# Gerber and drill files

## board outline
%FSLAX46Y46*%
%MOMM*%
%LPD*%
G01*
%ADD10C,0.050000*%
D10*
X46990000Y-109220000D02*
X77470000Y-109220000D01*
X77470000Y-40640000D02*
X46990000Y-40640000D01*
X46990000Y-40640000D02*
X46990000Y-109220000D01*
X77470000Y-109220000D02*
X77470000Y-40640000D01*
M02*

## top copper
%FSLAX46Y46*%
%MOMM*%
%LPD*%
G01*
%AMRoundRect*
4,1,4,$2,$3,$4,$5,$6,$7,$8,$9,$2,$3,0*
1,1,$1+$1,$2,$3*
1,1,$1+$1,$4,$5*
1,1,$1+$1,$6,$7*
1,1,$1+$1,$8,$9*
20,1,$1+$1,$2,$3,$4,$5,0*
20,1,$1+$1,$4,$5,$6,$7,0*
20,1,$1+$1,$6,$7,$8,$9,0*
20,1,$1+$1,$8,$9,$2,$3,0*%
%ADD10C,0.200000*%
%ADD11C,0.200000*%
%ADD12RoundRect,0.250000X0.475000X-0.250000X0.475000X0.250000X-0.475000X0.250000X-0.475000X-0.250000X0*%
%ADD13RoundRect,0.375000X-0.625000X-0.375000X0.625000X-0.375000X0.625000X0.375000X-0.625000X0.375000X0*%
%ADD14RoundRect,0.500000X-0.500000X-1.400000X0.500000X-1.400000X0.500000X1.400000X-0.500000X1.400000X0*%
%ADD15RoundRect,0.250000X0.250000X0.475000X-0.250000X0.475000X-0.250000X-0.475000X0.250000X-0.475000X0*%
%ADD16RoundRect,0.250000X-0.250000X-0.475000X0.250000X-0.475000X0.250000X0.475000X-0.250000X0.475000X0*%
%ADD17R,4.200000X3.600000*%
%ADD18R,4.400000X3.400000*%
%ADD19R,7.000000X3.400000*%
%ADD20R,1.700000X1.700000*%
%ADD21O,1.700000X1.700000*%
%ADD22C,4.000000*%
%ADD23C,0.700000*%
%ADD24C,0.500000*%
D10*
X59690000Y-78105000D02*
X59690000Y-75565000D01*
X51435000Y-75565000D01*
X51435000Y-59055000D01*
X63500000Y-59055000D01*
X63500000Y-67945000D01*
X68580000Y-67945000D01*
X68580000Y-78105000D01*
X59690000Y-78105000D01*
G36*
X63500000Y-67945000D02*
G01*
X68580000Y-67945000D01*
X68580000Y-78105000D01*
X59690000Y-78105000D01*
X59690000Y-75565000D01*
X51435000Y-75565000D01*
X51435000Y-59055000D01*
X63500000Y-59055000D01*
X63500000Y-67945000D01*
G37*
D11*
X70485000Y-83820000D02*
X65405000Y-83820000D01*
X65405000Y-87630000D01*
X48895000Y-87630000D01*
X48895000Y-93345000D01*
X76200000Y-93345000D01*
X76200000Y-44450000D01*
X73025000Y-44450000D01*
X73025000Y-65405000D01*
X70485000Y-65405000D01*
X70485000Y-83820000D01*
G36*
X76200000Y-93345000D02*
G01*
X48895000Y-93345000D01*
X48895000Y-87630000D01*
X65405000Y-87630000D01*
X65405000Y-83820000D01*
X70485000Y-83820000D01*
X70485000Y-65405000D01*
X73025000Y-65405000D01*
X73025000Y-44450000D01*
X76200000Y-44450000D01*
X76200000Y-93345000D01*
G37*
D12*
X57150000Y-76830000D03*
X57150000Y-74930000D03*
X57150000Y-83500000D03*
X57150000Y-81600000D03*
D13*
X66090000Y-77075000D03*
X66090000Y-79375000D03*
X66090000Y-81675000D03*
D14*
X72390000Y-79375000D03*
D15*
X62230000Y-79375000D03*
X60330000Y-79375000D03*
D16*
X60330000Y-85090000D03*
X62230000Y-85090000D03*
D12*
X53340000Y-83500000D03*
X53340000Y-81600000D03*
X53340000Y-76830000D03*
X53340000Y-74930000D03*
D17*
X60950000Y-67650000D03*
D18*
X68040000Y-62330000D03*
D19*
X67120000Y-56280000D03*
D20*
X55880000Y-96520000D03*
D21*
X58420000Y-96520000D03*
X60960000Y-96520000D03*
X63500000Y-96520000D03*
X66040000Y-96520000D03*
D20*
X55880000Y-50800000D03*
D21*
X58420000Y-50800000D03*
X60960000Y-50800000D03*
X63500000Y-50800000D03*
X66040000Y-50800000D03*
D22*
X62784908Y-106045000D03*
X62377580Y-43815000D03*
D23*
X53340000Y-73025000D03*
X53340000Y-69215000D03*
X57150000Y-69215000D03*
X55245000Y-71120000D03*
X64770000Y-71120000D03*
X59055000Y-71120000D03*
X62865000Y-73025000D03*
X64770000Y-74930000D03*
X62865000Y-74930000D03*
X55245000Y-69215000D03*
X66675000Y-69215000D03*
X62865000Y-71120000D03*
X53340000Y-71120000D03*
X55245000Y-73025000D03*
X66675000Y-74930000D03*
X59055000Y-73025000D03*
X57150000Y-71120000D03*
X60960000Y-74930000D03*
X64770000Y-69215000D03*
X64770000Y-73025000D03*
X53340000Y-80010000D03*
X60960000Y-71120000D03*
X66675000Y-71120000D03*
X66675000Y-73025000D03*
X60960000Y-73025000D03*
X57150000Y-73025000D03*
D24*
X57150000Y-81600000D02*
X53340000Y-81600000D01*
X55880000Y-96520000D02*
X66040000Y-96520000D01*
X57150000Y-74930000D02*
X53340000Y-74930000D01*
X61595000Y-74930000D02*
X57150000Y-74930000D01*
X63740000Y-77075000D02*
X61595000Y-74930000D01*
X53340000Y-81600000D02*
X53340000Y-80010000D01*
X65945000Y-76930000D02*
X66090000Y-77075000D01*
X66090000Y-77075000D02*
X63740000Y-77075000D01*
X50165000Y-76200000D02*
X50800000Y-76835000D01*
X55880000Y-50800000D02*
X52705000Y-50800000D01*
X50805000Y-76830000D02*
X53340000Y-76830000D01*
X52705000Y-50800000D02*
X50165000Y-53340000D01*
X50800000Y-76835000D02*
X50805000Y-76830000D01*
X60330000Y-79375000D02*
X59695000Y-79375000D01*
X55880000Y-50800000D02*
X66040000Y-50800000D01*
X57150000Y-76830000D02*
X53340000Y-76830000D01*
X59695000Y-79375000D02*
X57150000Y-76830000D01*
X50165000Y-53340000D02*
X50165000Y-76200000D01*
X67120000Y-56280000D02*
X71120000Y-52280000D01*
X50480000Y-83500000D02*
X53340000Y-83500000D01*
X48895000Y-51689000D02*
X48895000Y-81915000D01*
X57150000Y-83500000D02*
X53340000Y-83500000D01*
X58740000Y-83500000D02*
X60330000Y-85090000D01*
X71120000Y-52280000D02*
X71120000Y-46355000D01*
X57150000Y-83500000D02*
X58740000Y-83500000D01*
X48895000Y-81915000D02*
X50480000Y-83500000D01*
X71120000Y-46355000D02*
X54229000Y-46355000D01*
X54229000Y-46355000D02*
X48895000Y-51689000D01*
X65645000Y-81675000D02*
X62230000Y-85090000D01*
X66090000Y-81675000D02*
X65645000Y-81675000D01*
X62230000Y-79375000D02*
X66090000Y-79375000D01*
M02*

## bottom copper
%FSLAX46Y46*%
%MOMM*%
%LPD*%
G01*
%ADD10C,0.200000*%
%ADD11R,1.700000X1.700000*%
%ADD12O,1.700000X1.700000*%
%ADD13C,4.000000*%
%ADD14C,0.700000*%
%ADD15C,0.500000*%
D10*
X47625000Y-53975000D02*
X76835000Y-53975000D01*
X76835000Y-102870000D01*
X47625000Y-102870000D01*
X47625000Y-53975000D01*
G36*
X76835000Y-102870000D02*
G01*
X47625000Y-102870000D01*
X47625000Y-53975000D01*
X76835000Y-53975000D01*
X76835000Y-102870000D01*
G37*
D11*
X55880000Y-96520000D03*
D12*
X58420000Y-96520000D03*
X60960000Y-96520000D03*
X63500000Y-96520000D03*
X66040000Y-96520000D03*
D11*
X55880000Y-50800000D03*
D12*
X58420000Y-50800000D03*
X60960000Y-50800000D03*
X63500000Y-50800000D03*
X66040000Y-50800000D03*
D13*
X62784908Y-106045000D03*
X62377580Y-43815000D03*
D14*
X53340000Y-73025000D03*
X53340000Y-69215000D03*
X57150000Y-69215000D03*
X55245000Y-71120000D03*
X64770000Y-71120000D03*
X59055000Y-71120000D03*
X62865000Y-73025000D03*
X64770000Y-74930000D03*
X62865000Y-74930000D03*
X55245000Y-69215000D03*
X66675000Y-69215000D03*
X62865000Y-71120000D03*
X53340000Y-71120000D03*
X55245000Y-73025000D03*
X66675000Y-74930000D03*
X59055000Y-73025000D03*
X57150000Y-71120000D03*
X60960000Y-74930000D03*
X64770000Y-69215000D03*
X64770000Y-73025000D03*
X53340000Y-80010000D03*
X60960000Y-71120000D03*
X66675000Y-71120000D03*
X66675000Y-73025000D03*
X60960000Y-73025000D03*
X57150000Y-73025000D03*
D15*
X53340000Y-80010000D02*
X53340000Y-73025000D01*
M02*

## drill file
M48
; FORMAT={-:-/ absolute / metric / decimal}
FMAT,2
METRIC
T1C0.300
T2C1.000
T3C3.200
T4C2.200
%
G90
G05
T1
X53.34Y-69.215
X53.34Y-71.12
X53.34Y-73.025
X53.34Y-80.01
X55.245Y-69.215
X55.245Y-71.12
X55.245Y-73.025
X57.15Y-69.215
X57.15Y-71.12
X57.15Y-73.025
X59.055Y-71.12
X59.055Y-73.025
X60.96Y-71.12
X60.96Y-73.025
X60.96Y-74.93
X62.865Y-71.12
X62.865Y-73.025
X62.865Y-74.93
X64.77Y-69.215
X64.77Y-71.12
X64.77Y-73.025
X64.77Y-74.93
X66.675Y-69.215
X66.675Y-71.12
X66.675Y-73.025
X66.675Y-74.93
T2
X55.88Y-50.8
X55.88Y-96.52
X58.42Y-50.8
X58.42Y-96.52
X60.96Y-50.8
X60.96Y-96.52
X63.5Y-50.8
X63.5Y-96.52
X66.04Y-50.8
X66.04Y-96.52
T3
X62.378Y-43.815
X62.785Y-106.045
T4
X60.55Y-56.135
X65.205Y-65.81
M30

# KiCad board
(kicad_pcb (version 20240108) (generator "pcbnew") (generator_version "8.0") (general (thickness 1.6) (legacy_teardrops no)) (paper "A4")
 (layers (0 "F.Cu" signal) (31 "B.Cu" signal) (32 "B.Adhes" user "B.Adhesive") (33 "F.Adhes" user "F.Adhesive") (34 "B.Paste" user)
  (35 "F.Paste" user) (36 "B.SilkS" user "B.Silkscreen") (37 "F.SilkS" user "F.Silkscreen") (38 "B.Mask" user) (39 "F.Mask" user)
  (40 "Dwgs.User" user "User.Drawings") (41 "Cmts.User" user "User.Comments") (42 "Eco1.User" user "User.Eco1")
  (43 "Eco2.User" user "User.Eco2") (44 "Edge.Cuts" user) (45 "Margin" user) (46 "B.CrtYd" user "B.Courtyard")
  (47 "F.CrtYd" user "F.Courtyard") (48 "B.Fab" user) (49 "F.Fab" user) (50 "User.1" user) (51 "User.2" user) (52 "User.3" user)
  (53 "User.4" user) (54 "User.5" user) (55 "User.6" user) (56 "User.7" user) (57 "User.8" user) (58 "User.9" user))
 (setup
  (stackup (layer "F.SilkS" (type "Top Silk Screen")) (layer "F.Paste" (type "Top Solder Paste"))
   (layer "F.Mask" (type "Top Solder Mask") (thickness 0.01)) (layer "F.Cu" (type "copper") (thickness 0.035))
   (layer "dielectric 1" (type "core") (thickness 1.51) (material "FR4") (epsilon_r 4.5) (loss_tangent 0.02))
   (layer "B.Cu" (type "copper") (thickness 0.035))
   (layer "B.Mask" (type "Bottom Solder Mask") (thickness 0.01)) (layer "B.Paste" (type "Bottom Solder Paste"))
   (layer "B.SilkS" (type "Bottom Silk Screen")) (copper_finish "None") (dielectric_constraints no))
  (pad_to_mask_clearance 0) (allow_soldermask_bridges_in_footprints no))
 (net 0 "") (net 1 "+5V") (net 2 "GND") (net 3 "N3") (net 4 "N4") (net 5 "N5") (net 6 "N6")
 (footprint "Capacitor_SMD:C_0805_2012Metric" (layer "F.Cu") (at 57.15 75.88 90)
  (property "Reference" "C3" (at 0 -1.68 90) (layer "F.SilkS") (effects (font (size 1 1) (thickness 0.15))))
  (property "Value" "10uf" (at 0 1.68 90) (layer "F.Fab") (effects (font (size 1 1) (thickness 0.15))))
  (pad "1" smd roundrect (at -0.95 0 90) (size 1 1.45) (layers "F.Cu" "F.Paste" "F.Mask") (roundrect_rratio 0.25) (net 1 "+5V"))
  (pad "2" smd roundrect (at 0.95 0 90) (size 1 1.45) (layers "F.Cu" "F.Paste" "F.Mask") (roundrect_rratio 0.25) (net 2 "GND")))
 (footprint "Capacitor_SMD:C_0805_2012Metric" (layer "F.Cu") (at 57.15 82.55 90)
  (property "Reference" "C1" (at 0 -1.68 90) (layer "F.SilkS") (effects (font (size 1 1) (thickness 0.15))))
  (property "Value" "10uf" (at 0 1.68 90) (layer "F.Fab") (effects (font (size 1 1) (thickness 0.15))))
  (pad "1" smd roundrect (at -0.95 0 90) (size 1 1.45) (layers "F.Cu" "F.Paste" "F.Mask") (roundrect_rratio 0.25) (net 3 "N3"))
  (pad "2" smd roundrect (at 0.95 0 90) (size 1 1.45) (layers "F.Cu" "F.Paste" "F.Mask") (roundrect_rratio 0.25) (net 2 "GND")))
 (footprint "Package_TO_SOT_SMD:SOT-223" (layer "F.Cu") (at 69.24 79.375)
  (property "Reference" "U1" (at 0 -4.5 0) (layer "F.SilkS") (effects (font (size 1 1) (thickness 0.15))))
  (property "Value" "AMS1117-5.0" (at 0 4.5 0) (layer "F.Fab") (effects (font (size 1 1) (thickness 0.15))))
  (pad "1" smd roundrect (at -3.15 -2.3) (size 2 1.5) (layers "F.Cu" "F.Paste" "F.Mask") (roundrect_rratio 0.25) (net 2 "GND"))
  (pad "2" smd roundrect (at -3.15 0) (size 2 1.5) (layers "F.Cu" "F.Paste" "F.Mask") (roundrect_rratio 0.25) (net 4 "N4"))
  (pad "3" smd roundrect (at -3.15 2.3) (size 2 1.5) (layers "F.Cu" "F.Paste" "F.Mask") (roundrect_rratio 0.25) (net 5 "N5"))
  (pad "4" smd roundrect (at 3.15 0) (size 2 3.8) (layers "F.Cu" "F.Paste" "F.Mask") (roundrect_rratio 0.25)))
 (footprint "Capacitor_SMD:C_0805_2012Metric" (layer "F.Cu") (at 61.28 79.375 180)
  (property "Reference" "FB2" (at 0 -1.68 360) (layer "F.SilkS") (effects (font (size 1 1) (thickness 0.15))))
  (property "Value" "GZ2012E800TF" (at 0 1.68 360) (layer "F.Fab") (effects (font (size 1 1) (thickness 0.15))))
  (pad "1" smd roundrect (at -0.95 0 180) (size 1 1.45) (layers "F.Cu" "F.Paste" "F.Mask") (roundrect_rratio 0.25) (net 4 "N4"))
  (pad "2" smd roundrect (at 0.95 0 180) (size 1 1.45) (layers "F.Cu" "F.Paste" "F.Mask") (roundrect_rratio 0.25) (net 1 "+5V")))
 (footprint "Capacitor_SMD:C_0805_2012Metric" (layer "F.Cu") (at 61.28 85.09)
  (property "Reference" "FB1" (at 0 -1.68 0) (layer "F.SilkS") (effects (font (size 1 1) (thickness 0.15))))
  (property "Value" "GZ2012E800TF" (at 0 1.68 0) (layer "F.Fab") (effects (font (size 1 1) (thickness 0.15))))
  (pad "1" smd roundrect (at -0.95 0) (size 1 1.45) (layers "F.Cu" "F.Paste" "F.Mask") (roundrect_rratio 0.25) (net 3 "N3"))
  (pad "2" smd roundrect (at 0.95 0) (size 1 1.45) (layers "F.Cu" "F.Paste" "F.Mask") (roundrect_rratio 0.25) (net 5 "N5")))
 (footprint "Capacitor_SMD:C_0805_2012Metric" (layer "F.Cu") (at 53.34 82.55 90)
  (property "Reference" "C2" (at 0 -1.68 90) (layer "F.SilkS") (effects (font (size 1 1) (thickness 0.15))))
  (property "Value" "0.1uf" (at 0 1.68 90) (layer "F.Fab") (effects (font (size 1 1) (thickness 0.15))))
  (pad "1" smd roundrect (at -0.95 0 90) (size 1 1.45) (layers "F.Cu" "F.Paste" "F.Mask") (roundrect_rratio 0.25) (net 3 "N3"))
  (pad "2" smd roundrect (at 0.95 0 90) (size 1 1.45) (layers "F.Cu" "F.Paste" "F.Mask") (roundrect_rratio 0.25) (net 2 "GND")))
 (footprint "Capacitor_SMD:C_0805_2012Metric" (layer "F.Cu") (at 53.34 75.88 90)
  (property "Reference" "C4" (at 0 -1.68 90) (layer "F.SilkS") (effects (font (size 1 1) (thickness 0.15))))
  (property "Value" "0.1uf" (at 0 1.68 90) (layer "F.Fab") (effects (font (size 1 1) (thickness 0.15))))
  (pad "1" smd roundrect (at -0.95 0 90) (size 1 1.45) (layers "F.Cu" "F.Paste" "F.Mask") (roundrect_rratio 0.25) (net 1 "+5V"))
  (pad "2" smd roundrect (at 0.95 0 90) (size 1 1.45) (layers "F.Cu" "F.Paste" "F.Mask") (roundrect_rratio 0.25) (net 2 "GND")))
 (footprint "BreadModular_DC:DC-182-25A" (layer "F.Cu") (at 68.37 57.67 180)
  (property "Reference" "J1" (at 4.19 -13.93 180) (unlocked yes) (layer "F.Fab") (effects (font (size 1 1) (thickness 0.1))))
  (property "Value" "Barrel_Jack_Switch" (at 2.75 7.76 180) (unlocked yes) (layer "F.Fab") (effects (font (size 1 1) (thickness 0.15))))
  (pad "" np_thru_hole circle (at 3.165 -8.14 90) (size 2.2 2.2) (drill 2.2) (layers "F&B.Cu" "*.Mask"))
  (pad "" np_thru_hole circle (at 7.82 1.535 90) (size 2.2 2.2) (drill 2.2) (layers "F&B.Cu" "*.Mask"))
  (pad "1" smd rect (at 7.42 -9.98 90) (size 3.6 4.2) (layers "F.Cu" "F.Paste" "F.Mask") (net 2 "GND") (thermal_bridge_angle 45))
  (pad "2" smd rect (at 0.33 -4.66 90) (size 3.4 4.4) (layers "F.Cu" "F.Paste" "F.Mask") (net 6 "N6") (thermal_bridge_angle 45))
  (pad "3" smd rect (at 1.25 1.39 90) (size 3.4 7) (layers "F.Cu" "F.Paste" "F.Mask") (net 3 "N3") (thermal_bridge_angle 45)))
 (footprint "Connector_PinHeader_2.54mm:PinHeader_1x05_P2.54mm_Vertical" (layer "B.Cu") (at 55.88 96.52 -90)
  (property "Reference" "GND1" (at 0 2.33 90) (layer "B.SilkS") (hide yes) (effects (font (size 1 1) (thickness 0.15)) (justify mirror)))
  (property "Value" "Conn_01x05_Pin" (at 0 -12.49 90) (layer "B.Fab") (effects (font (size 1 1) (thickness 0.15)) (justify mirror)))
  (pad "1" thru_hole rect (at 0 0 270) (size 1.7 1.7) (drill 1) (layers "*.Cu" "*.Mask") (remove_unused_layers no) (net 2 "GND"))
  (pad "2" thru_hole oval (at 0 -2.54 270) (size 1.7 1.7) (drill 1) (layers "*.Cu" "*.Mask") (remove_unused_layers no) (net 2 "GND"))
  (pad "3" thru_hole oval (at 0 -5.08 270) (size 1.7 1.7) (drill 1) (layers "*.Cu" "*.Mask") (remove_unused_layers no) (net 2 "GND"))
  (pad "4" thru_hole oval (at 0 -7.62 270) (size 1.7 1.7) (drill 1) (layers "*.Cu" "*.Mask") (remove_unused_layers no) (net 2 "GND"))
  (pad "5" thru_hole oval (at 0 -10.16 270) (size 1.7 1.7) (drill 1) (layers "*.Cu" "*.Mask") (remove_unused_layers no) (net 2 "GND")))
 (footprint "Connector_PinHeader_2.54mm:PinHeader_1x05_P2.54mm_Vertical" (layer "B.Cu") (at 55.88 50.8 -90)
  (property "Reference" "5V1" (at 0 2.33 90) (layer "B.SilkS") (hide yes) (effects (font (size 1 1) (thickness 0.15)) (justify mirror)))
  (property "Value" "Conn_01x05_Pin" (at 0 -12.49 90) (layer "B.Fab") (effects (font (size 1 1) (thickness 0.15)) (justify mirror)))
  (pad "1" thru_hole rect (at 0 0 270) (size 1.7 1.7) (drill 1) (layers "*.Cu" "*.Mask") (remove_unused_layers no) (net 1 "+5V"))
  (pad "2" thru_hole oval (at 0 -2.54 270) (size 1.7 1.7) (drill 1) (layers "*.Cu" "*.Mask") (remove_unused_layers no) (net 1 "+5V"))
  (pad "3" thru_hole oval (at 0 -5.08 270) (size 1.7 1.7) (drill 1) (layers "*.Cu" "*.Mask") (remove_unused_layers no) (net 1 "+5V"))
  (pad "4" thru_hole oval (at 0 -7.62 270) (size 1.7 1.7) (drill 1) (layers "*.Cu" "*.Mask") (remove_unused_layers no) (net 1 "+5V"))
  (pad "5" thru_hole oval (at 0 -10.16 270) (size 1.7 1.7) (drill 1) (layers "*.Cu" "*.Mask") (remove_unused_layers no) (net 1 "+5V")))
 (gr_poly
  (pts (xy 59.69 78.105) (xy 59.69 75.565) (xy 51.435 75.565) (xy 51.435 59.055) (xy 63.5 59.055) (xy 63.5 67.945) (xy 68.58 67.945)
   (xy 68.58 78.105))
  (stroke (width 0.2) (type solid)) (fill solid) (layer "F.Cu") (net 2))
 (gr_poly
  (pts (xy 70.485 83.82) (xy 65.405 83.82) (xy 65.405 87.63) (xy 48.895 87.63) (xy 48.895 93.345) (xy 76.2 93.345) (xy 76.2 44.45)
   (xy 73.025 44.45) (xy 73.025 65.405) (xy 70.485 65.405))
  (stroke (width 0.2) (type solid)) (fill solid) (layer "F.Cu"))
 (gr_poly
  (pts (xy 47.625 53.975) (xy 76.835 53.975) (xy 76.835 102.87) (xy 47.625 102.87)) (stroke (width 0.2) (type solid)) (fill solid)
  (layer "B.Cu") (net 2))
 (gr_line (start 46.99 109.22) (end 77.47 109.22) (stroke (width 0.05) (type default)) (layer "Edge.Cuts"))
 (gr_line (start 77.47 40.64) (end 46.99 40.64) (stroke (width 0.05) (type default)) (layer "Edge.Cuts"))
 (gr_line (start 46.99 40.64) (end 46.99 109.22) (stroke (width 0.05) (type default)) (layer "Edge.Cuts"))
 (gr_line (start 77.47 109.22) (end 77.47 40.64) (stroke (width 0.05) (type default)) (layer "Edge.Cuts"))
 (via (at 62.784908 106.045) (size 4) (drill 3.2) (layers "F.Cu" "B.Cu") (free yes) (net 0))
 (via (at 62.37758 43.815) (size 4) (drill 3.2) (layers "F.Cu" "B.Cu") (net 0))
 (segment (start 57.15 81.6) (end 53.34 81.6) (width 0.5) (layer "F.Cu") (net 2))
 (segment (start 55.88 96.52) (end 66.04 96.52) (width 0.5) (layer "F.Cu") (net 2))
 (segment (start 57.15 74.93) (end 53.34 74.93) (width 0.5) (layer "F.Cu") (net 2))
 (segment (start 61.595 74.93) (end 57.15 74.93) (width 0.5) (layer "F.Cu") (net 2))
 (segment (start 63.74 77.075) (end 61.595 74.93) (width 0.5) (layer "F.Cu") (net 2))
 (segment (start 53.34 81.6) (end 53.34 80.01) (width 0.5) (layer "F.Cu") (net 2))
 (segment (start 65.945 76.93) (end 66.09 77.075) (width 0.5) (layer "F.Cu") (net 2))
 (segment (start 66.09 77.075) (end 63.74 77.075) (width 0.5) (layer "F.Cu") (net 2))
 (via (at 53.34 73.025) (size 0.7) (drill 0.3) (layers "F.Cu" "B.Cu") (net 2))
 (via (at 53.34 69.215) (size 0.7) (drill 0.3) (layers "F.Cu" "B.Cu") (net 2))
 (via (at 57.15 69.215) (size 0.7) (drill 0.3) (layers "F.Cu" "B.Cu") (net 2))
 (via (at 55.245 71.12) (size 0.7) (drill 0.3) (layers "F.Cu" "B.Cu") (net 2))
 (via (at 64.77 71.12) (size 0.7) (drill 0.3) (layers "F.Cu" "B.Cu") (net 2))
 (via (at 59.055 71.12) (size 0.7) (drill 0.3) (layers "F.Cu" "B.Cu") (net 2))
 (via (at 62.865 73.025) (size 0.7) (drill 0.3) (layers "F.Cu" "B.Cu") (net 2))
 (via (at 64.77 74.93) (size 0.7) (drill 0.3) (layers "F.Cu" "B.Cu") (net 2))
 (via (at 62.865 74.93) (size 0.7) (drill 0.3) (layers "F.Cu" "B.Cu") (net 2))
 (via (at 55.245 69.215) (size 0.7) (drill 0.3) (layers "F.Cu" "B.Cu") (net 2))
 (via (at 66.675 69.215) (size 0.7) (drill 0.3) (layers "F.Cu" "B.Cu") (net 2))
 (via (at 62.865 71.12) (size 0.7) (drill 0.3) (layers "F.Cu" "B.Cu") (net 2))
 (via (at 53.34 71.12) (size 0.7) (drill 0.3) (layers "F.Cu" "B.Cu") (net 2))
 (via (at 55.245 73.025) (size 0.7) (drill 0.3) (layers "F.Cu" "B.Cu") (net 2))
 (via (at 66.675 74.93) (size 0.7) (drill 0.3) (layers "F.Cu" "B.Cu") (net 2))
 (via (at 59.055 73.025) (size 0.7) (drill 0.3) (layers "F.Cu" "B.Cu") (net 2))
 (via (at 57.15 71.12) (size 0.7) (drill 0.3) (layers "F.Cu" "B.Cu") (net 2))
 (via (at 60.96 74.93) (size 0.7) (drill 0.3) (layers "F.Cu" "B.Cu") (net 2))
 (via (at 64.77 69.215) (size 0.7) (drill 0.3) (layers "F.Cu" "B.Cu") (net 2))
 (via (at 64.77 73.025) (size 0.7) (drill 0.3) (layers "F.Cu" "B.Cu") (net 2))
 (via (at 53.34 80.01) (size 0.7) (drill 0.3) (layers "F.Cu" "B.Cu") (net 2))
 (via (at 60.96 71.12) (size 0.7) (drill 0.3) (layers "F.Cu" "B.Cu") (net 2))
 (via (at 66.675 71.12) (size 0.7) (drill 0.3) (layers "F.Cu" "B.Cu") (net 2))
 (via (at 66.675 73.025) (size 0.7) (drill 0.3) (layers "F.Cu" "B.Cu") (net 2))
 (via (at 60.96 73.025) (size 0.7) (drill 0.3) (layers "F.Cu" "B.Cu") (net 2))
 (via (at 57.15 73.025) (size 0.7) (drill 0.3) (layers "F.Cu" "B.Cu") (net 2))
 (segment (start 53.34 80.01) (end 53.34 73.025) (width 0.5) (layer "B.Cu") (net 2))
 (segment (start 50.165 76.2) (end 50.8 76.835) (width 0.5) (layer "F.Cu") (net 1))
 (segment (start 55.88 50.8) (end 52.705 50.8) (width 0.5) (layer "F.Cu") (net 1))
 (segment (start 50.805 76.83) (end 53.34 76.83) (width 0.5) (layer "F.Cu") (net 1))
 (segment (start 52.705 50.8) (end 50.165 53.34) (width 0.5) (layer "F.Cu") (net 1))
 (segment (start 50.8 76.835) (end 50.805 76.83) (width 0.5) (layer "F.Cu") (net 1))
 (segment (start 60.33 79.375) (end 59.695 79.375) (width 0.5) (layer "F.Cu") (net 1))
 (segment (start 55.88 50.8) (end 66.04 50.8) (width 0.5) (layer "F.Cu") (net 1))
 (segment (start 57.15 76.83) (end 53.34 76.83) (width 0.5) (layer "F.Cu") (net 1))
 (segment (start 59.695 79.375) (end 57.15 76.83) (width 0.5) (layer "F.Cu") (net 1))
 (segment (start 50.165 53.34) (end 50.165 76.2) (width 0.5) (layer "F.Cu") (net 1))
 (segment (start 67.12 56.28) (end 71.12 52.28) (width 0.5) (layer "F.Cu") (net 3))
 (segment (start 50.48 83.5) (end 53.34 83.5) (width 0.5) (layer "F.Cu") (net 3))
 (segment (start 48.895 51.689) (end 48.895 81.915) (width 0.5) (layer "F.Cu") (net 3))
 (segment (start 57.15 83.5) (end 53.34 83.5) (width 0.5) (layer "F.Cu") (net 3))
 (segment (start 58.74 83.5) (end 60.33 85.09) (width 0.5) (layer "F.Cu") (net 3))
 (segment (start 71.12 52.28) (end 71.12 46.355) (width 0.5) (layer "F.Cu") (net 3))
 (segment (start 57.15 83.5) (end 58.74 83.5) (width 0.5) (layer "F.Cu") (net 3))
 (segment (start 48.895 81.915) (end 50.48 83.5) (width 0.5) (layer "F.Cu") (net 3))
 (segment (start 71.12 46.355) (end 54.229 46.355) (width 0.5) (layer "F.Cu") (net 3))
 (segment (start 54.229 46.355) (end 48.895 51.689) (width 0.5) (layer "F.Cu") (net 3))
 (segment (start 65.645 81.675) (end 62.23 85.09) (width 0.5) (layer "F.Cu") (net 5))
 (segment (start 66.09 81.675) (end 65.645 81.675) (width 0.5) (layer "F.Cu") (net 5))
 (segment (start 62.23 79.375) (end 66.09 79.375) (width 0.5) (layer "F.Cu") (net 4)))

